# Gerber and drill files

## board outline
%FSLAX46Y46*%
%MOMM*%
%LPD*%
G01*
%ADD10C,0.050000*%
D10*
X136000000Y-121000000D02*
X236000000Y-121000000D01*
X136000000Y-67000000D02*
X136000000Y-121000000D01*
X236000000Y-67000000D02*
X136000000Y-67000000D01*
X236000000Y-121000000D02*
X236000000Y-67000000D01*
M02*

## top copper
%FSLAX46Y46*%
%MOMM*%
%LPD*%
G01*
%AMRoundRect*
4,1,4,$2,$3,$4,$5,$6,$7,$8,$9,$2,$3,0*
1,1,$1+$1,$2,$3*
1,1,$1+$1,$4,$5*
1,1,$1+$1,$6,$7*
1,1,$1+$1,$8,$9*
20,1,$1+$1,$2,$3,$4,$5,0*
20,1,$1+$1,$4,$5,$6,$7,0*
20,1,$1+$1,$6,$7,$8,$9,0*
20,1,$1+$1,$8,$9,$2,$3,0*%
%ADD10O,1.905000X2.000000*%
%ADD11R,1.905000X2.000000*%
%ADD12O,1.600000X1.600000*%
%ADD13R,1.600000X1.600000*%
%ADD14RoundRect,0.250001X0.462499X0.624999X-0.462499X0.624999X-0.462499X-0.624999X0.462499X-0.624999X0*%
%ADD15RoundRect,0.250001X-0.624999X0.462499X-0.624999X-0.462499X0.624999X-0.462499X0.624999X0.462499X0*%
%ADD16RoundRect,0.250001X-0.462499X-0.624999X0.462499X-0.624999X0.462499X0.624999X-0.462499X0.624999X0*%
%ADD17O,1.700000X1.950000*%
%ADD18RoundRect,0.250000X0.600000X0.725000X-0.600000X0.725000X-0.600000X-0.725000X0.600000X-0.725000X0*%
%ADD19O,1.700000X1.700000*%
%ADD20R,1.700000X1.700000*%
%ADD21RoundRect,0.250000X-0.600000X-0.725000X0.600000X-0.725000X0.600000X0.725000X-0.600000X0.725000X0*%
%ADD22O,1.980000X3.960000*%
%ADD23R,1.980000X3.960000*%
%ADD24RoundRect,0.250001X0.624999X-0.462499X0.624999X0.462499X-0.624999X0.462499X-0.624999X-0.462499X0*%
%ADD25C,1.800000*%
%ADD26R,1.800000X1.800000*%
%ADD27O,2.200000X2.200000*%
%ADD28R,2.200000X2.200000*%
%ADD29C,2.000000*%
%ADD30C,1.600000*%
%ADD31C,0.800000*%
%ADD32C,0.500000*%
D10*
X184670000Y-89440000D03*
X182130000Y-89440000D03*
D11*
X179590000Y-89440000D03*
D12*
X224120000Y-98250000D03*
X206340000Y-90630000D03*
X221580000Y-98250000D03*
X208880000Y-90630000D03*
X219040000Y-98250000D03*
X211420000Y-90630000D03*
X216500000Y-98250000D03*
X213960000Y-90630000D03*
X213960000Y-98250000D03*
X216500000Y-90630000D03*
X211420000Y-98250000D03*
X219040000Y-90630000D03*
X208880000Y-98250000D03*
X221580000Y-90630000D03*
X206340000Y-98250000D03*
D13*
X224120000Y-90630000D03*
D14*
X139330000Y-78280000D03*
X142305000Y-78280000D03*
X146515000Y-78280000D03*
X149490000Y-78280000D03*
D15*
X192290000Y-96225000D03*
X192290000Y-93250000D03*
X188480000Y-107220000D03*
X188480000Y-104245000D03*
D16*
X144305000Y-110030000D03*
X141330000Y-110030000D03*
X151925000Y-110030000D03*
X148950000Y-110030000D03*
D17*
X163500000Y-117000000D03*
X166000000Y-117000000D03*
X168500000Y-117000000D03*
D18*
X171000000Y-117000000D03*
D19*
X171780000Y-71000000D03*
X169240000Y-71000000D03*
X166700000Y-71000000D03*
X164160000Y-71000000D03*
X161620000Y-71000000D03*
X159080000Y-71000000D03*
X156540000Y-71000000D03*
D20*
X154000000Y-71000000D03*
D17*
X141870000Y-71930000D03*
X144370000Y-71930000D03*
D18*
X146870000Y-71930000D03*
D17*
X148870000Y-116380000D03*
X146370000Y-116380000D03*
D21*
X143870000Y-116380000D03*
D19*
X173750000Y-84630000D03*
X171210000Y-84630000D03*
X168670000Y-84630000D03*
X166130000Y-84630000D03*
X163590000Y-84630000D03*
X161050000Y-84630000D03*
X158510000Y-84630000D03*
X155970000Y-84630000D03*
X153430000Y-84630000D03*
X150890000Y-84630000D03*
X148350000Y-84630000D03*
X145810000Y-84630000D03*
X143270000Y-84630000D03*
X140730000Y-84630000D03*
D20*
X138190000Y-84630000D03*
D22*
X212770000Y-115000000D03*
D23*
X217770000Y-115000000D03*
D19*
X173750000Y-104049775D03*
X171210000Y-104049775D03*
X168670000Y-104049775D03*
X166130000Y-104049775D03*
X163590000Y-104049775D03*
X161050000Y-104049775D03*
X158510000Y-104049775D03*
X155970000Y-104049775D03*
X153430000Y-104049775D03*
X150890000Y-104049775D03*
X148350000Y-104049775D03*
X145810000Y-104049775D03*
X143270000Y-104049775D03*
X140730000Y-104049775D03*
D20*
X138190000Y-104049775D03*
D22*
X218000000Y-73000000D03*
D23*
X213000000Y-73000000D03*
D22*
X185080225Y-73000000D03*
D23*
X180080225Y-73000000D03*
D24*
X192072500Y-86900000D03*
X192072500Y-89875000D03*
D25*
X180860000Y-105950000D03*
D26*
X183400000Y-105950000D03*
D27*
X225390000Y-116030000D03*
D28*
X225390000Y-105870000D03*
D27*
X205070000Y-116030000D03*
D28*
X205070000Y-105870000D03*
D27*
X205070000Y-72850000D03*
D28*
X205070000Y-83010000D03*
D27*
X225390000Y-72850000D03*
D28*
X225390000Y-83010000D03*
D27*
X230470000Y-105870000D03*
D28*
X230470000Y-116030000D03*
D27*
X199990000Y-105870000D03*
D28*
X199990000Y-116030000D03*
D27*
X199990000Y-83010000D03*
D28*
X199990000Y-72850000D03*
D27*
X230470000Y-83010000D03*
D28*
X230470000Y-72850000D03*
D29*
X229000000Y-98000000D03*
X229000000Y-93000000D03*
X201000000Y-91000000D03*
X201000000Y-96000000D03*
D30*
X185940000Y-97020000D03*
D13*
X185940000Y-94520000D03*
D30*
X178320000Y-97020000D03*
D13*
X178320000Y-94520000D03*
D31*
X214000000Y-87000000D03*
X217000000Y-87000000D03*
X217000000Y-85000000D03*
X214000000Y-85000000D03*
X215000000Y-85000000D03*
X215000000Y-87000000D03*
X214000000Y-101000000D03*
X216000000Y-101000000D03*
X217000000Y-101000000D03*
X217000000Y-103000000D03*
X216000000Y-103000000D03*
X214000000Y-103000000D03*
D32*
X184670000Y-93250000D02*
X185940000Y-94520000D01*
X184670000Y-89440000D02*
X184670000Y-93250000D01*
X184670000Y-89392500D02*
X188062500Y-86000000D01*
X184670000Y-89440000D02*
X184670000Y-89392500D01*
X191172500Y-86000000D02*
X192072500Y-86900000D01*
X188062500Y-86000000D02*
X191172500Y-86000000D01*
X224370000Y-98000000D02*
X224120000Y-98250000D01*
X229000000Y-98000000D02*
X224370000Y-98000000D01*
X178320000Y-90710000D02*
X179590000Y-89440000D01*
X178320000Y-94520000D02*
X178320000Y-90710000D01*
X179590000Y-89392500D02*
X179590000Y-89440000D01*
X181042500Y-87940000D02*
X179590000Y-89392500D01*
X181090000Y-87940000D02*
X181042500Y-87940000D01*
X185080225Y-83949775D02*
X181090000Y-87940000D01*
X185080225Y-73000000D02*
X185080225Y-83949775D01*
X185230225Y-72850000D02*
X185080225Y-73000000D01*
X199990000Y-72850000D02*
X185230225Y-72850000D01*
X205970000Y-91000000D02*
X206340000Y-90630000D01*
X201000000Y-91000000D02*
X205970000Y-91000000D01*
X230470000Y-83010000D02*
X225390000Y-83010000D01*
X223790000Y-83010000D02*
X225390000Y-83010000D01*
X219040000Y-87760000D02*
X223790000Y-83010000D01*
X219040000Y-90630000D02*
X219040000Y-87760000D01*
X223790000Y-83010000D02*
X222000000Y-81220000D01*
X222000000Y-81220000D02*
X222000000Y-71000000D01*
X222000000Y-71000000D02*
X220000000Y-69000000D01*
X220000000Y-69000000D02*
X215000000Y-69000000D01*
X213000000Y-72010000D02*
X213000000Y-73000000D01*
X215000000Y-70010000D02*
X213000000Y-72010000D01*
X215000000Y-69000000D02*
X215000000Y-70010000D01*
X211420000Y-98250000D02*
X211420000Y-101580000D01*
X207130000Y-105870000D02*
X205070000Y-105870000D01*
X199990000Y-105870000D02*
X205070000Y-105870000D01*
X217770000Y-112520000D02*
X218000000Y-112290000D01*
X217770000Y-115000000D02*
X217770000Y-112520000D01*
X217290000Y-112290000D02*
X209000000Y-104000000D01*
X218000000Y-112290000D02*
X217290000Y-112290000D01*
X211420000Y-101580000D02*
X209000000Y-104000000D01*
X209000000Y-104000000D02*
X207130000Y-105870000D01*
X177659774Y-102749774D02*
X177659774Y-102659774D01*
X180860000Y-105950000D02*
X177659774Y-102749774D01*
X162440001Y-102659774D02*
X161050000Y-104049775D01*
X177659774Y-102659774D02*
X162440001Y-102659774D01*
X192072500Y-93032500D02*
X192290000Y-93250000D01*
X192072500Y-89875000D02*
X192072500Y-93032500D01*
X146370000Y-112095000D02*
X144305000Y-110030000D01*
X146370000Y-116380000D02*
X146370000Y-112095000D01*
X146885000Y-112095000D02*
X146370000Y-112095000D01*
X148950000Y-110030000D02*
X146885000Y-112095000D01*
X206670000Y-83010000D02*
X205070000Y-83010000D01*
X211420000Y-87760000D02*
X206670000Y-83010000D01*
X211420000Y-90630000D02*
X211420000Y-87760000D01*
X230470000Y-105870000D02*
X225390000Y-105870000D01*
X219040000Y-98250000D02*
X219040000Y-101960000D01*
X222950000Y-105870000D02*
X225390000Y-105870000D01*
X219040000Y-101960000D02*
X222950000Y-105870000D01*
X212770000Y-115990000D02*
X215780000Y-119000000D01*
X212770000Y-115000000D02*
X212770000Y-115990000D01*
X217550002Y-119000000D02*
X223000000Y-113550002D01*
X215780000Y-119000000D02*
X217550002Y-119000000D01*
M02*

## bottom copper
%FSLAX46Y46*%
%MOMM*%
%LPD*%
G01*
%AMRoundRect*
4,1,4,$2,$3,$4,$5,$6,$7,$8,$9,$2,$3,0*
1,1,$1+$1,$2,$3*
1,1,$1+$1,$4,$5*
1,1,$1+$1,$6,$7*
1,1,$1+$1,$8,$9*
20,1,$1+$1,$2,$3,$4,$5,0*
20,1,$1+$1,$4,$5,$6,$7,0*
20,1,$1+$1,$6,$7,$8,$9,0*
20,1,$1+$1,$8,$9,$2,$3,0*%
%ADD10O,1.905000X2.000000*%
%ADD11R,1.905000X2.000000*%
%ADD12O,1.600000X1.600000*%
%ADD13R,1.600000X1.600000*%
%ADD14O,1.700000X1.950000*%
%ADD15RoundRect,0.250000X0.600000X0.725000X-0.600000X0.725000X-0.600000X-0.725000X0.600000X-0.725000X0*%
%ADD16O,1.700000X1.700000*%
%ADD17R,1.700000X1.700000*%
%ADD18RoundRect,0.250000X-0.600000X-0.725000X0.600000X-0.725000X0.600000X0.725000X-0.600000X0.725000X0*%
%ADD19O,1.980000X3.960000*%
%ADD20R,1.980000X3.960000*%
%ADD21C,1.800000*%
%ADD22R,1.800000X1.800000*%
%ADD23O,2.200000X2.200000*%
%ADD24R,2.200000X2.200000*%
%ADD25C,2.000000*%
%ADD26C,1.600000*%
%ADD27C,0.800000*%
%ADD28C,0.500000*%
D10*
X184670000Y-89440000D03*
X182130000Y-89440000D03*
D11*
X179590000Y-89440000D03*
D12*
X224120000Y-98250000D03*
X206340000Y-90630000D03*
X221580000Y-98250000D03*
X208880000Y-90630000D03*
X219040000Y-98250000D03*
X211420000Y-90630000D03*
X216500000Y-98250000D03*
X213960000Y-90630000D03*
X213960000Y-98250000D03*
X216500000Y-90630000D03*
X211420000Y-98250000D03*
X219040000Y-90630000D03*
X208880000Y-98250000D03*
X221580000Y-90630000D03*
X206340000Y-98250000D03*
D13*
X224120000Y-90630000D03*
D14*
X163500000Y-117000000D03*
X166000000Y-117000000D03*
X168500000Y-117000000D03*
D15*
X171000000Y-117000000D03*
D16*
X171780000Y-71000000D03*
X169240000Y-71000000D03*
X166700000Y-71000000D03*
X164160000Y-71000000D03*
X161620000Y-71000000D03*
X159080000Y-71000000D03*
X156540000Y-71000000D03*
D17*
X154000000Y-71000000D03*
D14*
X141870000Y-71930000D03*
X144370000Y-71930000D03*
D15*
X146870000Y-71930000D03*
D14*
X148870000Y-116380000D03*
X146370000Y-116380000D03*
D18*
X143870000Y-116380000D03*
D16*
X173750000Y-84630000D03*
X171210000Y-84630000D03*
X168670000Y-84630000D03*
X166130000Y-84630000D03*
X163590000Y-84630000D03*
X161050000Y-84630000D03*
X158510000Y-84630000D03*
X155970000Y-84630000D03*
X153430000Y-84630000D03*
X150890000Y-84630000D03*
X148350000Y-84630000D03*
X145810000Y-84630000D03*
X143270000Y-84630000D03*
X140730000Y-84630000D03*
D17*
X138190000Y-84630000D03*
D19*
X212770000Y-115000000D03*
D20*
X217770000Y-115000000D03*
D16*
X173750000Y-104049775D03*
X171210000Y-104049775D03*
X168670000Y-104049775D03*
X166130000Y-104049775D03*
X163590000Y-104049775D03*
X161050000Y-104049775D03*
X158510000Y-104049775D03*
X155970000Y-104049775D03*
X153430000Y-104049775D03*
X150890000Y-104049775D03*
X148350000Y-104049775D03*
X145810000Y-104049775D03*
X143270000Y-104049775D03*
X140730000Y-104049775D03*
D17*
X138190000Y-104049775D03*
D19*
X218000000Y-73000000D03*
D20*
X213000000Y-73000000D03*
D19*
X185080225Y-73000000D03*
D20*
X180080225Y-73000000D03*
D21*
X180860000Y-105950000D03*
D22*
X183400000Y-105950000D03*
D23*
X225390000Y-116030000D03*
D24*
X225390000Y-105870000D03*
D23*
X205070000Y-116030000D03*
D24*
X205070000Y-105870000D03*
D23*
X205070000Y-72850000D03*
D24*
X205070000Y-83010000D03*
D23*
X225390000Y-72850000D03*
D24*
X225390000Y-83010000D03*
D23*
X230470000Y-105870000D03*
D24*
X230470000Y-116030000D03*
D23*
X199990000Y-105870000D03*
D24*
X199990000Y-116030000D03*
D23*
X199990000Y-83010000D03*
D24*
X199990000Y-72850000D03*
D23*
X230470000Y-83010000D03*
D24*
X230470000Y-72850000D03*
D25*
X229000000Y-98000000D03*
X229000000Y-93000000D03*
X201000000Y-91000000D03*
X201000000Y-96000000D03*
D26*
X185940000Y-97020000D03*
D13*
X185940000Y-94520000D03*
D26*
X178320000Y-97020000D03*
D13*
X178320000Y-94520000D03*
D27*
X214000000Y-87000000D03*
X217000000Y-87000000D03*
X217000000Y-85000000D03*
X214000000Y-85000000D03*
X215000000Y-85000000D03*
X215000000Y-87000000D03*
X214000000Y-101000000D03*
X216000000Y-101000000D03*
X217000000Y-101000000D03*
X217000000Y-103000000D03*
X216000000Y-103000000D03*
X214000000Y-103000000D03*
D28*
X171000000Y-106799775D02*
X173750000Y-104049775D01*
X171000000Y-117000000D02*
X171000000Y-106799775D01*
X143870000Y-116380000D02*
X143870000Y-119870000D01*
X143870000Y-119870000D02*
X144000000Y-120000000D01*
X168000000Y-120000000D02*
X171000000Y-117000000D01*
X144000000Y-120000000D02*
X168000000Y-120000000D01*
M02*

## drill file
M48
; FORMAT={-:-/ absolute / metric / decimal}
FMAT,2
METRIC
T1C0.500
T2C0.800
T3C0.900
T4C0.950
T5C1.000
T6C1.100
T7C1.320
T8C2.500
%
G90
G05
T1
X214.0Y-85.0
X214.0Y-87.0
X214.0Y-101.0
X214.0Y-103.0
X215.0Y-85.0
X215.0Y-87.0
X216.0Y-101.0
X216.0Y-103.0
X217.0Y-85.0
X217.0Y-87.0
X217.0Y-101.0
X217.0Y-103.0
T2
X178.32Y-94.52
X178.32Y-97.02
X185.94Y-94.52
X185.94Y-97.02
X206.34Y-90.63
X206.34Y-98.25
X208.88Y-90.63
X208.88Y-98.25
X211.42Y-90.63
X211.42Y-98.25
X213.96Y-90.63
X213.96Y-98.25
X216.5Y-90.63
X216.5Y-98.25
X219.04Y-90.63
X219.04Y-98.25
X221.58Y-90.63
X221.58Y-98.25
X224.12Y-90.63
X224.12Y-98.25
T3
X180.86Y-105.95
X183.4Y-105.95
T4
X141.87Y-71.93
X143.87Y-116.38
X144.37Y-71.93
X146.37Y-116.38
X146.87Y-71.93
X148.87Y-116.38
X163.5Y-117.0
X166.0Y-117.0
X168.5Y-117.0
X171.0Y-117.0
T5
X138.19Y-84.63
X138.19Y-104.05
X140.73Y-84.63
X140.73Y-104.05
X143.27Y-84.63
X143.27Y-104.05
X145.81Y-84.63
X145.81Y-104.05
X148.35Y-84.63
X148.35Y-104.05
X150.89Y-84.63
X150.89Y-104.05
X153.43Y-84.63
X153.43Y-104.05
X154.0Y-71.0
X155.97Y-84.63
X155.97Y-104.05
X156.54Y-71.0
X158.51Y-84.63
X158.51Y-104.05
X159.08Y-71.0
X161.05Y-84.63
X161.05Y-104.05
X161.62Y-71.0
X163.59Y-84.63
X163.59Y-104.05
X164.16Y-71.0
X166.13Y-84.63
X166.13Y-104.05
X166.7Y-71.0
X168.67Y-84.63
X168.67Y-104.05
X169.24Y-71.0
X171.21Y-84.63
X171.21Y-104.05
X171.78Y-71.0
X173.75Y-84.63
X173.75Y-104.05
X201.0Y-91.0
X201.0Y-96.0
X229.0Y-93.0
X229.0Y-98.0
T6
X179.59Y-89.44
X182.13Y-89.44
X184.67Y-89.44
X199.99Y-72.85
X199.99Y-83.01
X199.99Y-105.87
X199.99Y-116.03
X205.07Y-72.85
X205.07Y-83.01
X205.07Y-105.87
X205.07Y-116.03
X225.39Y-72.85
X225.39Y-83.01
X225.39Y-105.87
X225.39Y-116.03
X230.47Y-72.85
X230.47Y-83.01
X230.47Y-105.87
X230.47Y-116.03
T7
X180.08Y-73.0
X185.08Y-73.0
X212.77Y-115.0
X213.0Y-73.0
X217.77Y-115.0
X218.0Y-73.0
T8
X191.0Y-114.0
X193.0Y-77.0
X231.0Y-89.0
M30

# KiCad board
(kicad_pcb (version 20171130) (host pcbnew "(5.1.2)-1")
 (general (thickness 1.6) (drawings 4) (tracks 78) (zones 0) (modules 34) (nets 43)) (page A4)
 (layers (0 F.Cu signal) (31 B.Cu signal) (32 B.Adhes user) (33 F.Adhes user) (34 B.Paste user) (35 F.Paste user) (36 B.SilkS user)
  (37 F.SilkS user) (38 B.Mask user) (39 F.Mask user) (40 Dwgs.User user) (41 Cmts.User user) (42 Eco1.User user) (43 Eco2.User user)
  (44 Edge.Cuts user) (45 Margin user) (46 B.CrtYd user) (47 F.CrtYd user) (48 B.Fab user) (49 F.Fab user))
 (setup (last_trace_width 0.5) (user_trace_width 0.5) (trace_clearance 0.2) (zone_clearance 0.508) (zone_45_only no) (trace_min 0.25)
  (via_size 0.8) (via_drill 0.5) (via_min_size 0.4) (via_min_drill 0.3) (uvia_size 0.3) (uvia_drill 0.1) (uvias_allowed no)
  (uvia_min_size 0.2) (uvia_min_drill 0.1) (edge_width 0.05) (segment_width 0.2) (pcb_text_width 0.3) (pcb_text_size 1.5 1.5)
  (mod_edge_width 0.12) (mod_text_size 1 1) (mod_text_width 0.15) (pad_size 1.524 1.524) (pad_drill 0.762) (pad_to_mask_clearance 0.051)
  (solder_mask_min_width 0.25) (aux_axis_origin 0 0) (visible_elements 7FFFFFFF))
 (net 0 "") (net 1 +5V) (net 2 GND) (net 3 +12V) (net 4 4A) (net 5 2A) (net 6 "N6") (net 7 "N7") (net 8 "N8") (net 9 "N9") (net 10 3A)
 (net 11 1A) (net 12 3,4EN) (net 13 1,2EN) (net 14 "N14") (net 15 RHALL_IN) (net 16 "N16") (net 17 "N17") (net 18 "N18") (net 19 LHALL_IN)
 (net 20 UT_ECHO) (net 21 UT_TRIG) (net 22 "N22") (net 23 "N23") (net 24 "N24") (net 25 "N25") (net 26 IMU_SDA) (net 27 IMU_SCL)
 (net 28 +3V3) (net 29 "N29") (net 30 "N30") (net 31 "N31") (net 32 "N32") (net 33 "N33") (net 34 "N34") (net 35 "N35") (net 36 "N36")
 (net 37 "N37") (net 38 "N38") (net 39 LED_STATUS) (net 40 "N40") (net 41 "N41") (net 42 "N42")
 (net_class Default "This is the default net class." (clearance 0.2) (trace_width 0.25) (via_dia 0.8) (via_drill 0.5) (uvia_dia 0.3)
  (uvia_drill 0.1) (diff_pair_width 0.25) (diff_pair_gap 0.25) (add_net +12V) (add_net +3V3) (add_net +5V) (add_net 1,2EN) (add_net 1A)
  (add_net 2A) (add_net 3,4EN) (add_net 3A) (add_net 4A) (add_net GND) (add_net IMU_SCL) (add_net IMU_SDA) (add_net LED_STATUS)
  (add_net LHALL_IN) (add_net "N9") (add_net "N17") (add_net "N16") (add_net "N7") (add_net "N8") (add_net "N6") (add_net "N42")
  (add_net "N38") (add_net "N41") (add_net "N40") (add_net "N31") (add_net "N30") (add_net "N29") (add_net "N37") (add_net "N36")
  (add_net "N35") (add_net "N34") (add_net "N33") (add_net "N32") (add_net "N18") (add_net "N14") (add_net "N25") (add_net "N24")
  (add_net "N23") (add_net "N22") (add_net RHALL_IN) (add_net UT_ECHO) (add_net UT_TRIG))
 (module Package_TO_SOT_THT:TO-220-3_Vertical (layer F.Cu) (at 179.59 89.44)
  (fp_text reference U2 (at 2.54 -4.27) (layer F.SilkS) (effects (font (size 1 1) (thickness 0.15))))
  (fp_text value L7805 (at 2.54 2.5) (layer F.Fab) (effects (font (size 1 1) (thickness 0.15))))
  (pad 3 thru_hole oval (at 5.08 0) (size 1.905 2) (drill 1.1) (layers *.Cu *.Mask) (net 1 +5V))
  (pad 2 thru_hole oval (at 2.54 0) (size 1.905 2) (drill 1.1) (layers *.Cu *.Mask) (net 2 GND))
  (pad 1 thru_hole rect (at 0 0) (size 1.905 2) (drill 1.1) (layers *.Cu *.Mask) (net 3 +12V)))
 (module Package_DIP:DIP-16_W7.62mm (layer F.Cu) (at 224.12 90.63 270)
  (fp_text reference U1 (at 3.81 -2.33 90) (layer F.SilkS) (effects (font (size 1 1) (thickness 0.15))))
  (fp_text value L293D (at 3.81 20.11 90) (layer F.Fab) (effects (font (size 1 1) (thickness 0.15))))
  (pad 16 thru_hole oval (at 7.62 0 270) (size 1.6 1.6) (drill 0.8) (layers *.Cu *.Mask) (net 1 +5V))
  (pad 8 thru_hole oval (at 0 17.78 270) (size 1.6 1.6) (drill 0.8) (layers *.Cu *.Mask) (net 3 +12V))
  (pad 15 thru_hole oval (at 7.62 2.54 270) (size 1.6 1.6) (drill 0.8) (layers *.Cu *.Mask) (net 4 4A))
  (pad 7 thru_hole oval (at 0 15.24 270) (size 1.6 1.6) (drill 0.8) (layers *.Cu *.Mask) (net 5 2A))
  (pad 14 thru_hole oval (at 7.62 5.08 270) (size 1.6 1.6) (drill 0.8) (layers *.Cu *.Mask) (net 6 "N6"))
  (pad 6 thru_hole oval (at 0 12.7 270) (size 1.6 1.6) (drill 0.8) (layers *.Cu *.Mask) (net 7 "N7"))
  (pad 13 thru_hole oval (at 7.62 7.62 270) (size 1.6 1.6) (drill 0.8) (layers *.Cu *.Mask) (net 2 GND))
  (pad 5 thru_hole oval (at 0 10.16 270) (size 1.6 1.6) (drill 0.8) (layers *.Cu *.Mask) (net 2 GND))
  (pad 12 thru_hole oval (at 7.62 10.16 270) (size 1.6 1.6) (drill 0.8) (layers *.Cu *.Mask) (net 2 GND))
  (pad 4 thru_hole oval (at 0 7.62 270) (size 1.6 1.6) (drill 0.8) (layers *.Cu *.Mask) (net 2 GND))
  (pad 11 thru_hole oval (at 7.62 12.7 270) (size 1.6 1.6) (drill 0.8) (layers *.Cu *.Mask) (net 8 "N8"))
  (pad 3 thru_hole oval (at 0 5.08 270) (size 1.6 1.6) (drill 0.8) (layers *.Cu *.Mask) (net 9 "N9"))
  (pad 10 thru_hole oval (at 7.62 15.24 270) (size 1.6 1.6) (drill 0.8) (layers *.Cu *.Mask) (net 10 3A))
  (pad 2 thru_hole oval (at 0 2.54 270) (size 1.6 1.6) (drill 0.8) (layers *.Cu *.Mask) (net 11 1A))
  (pad 9 thru_hole oval (at 7.62 17.78 270) (size 1.6 1.6) (drill 0.8) (layers *.Cu *.Mask) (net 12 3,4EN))
  (pad 1 thru_hole rect (at 0 0 270) (size 1.6 1.6) (drill 0.8) (layers *.Cu *.Mask) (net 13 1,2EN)))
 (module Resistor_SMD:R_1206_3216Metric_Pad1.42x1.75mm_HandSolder (layer F.Cu) (at 140.8175 78.28 180)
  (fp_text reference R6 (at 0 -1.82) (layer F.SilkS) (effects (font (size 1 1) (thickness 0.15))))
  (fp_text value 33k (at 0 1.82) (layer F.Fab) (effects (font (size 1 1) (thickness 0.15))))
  (pad 2 smd roundrect (at 1.4875 0 180) (size 1.425 1.75) (layers F.Cu F.Paste F.Mask) (roundrect_rratio 0.175439) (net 2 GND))
  (pad 1 smd roundrect (at -1.4875 0 180) (size 1.425 1.75) (layers F.Cu F.Paste F.Mask) (roundrect_rratio 0.175439) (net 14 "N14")))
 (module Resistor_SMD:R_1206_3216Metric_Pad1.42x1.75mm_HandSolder (layer F.Cu) (at 148.0025 78.28 180)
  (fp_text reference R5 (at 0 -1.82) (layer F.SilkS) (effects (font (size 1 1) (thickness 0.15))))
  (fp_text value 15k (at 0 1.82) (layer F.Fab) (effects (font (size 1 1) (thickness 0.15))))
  (pad 2 smd roundrect (at 1.4875 0 180) (size 1.425 1.75) (layers F.Cu F.Paste F.Mask) (roundrect_rratio 0.175439) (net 14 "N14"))
  (pad 1 smd roundrect (at -1.4875 0 180) (size 1.425 1.75) (layers F.Cu F.Paste F.Mask) (roundrect_rratio 0.175439) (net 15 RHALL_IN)))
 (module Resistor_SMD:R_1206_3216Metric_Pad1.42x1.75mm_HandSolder (layer F.Cu) (at 192.29 94.7375 270)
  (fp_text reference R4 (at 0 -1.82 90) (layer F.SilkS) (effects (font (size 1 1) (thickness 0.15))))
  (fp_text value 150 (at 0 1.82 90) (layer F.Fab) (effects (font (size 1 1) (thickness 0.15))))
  (pad 2 smd roundrect (at 1.4875 0 270) (size 1.425 1.75) (layers F.Cu F.Paste F.Mask) (roundrect_rratio 0.175439) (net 2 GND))
  (pad 1 smd roundrect (at -1.4875 0 270) (size 1.425 1.75) (layers F.Cu F.Paste F.Mask) (roundrect_rratio 0.175439) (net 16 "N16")))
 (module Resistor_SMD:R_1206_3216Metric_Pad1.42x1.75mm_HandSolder (layer F.Cu) (at 188.48 105.7325 270)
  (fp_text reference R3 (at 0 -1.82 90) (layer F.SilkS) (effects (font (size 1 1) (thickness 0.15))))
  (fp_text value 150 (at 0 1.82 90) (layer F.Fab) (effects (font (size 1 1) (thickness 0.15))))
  (pad 2 smd roundrect (at 1.4875 0 270) (size 1.425 1.75) (layers F.Cu F.Paste F.Mask) (roundrect_rratio 0.175439) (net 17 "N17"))
  (pad 1 smd roundrect (at -1.4875 0 270) (size 1.425 1.75) (layers F.Cu F.Paste F.Mask) (roundrect_rratio 0.175439) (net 2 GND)))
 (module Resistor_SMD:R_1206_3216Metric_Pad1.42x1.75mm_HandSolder (layer F.Cu) (at 142.8175 110.03)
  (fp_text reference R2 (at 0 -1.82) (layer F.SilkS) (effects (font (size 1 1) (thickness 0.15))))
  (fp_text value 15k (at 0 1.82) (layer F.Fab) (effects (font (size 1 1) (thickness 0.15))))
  (pad 2 smd roundrect (at 1.4875 0) (size 1.425 1.75) (layers F.Cu F.Paste F.Mask) (roundrect_rratio 0.175439) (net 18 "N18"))
  (pad 1 smd roundrect (at -1.4875 0) (size 1.425 1.75) (layers F.Cu F.Paste F.Mask) (roundrect_rratio 0.175439) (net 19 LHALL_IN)))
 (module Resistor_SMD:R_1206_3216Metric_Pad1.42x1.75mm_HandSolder (layer F.Cu) (at 150.4375 110.03)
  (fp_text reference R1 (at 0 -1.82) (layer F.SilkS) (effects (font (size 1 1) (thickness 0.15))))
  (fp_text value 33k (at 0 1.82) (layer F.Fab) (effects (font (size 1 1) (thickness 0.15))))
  (pad 2 smd roundrect (at 1.4875 0) (size 1.425 1.75) (layers F.Cu F.Paste F.Mask) (roundrect_rratio 0.175439) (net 2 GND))
  (pad 1 smd roundrect (at -1.4875 0) (size 1.425 1.75) (layers F.Cu F.Paste F.Mask) (roundrect_rratio 0.175439) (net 18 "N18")))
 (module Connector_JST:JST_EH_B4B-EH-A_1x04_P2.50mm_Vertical (layer F.Cu) (at 171 117 180)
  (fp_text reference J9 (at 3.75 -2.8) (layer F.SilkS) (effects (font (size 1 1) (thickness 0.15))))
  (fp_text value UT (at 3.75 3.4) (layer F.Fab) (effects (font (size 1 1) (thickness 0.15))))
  (pad 4 thru_hole oval (at 7.5 0 180) (size 1.7 1.95) (drill 0.95) (layers *.Cu *.Mask) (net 2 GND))
  (pad 3 thru_hole oval (at 5 0 180) (size 1.7 1.95) (drill 0.95) (layers *.Cu *.Mask) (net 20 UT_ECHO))
  (pad 2 thru_hole oval (at 2.5 0 180) (size 1.7 1.95) (drill 0.95) (layers *.Cu *.Mask) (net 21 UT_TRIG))
  (pad 1 thru_hole roundrect (at 0 0 180) (size 1.7 1.95) (drill 0.95) (layers *.Cu *.Mask) (roundrect_rratio 0.147059) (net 1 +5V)))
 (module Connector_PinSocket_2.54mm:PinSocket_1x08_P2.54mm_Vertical (layer F.Cu) (at 154 71 90)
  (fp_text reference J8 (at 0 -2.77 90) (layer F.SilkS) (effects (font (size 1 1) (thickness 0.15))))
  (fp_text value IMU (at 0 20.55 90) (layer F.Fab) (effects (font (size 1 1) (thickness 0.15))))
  (pad 8 thru_hole oval (at 0 17.78 90) (size 1.7 1.7) (drill 1) (layers *.Cu *.Mask) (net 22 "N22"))
  (pad 7 thru_hole oval (at 0 15.24 90) (size 1.7 1.7) (drill 1) (layers *.Cu *.Mask) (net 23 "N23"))
  (pad 6 thru_hole oval (at 0 12.7 90) (size 1.7 1.7) (drill 1) (layers *.Cu *.Mask) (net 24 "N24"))
  (pad 5 thru_hole oval (at 0 10.16 90) (size 1.7 1.7) (drill 1) (layers *.Cu *.Mask) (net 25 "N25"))
  (pad 4 thru_hole oval (at 0 7.62 90) (size 1.7 1.7) (drill 1) (layers *.Cu *.Mask) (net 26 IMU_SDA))
  (pad 3 thru_hole oval (at 0 5.08 90) (size 1.7 1.7) (drill 1) (layers *.Cu *.Mask) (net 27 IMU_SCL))
  (pad 2 thru_hole oval (at 0 2.54 90) (size 1.7 1.7) (drill 1) (layers *.Cu *.Mask) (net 2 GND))
  (pad 1 thru_hole rect (at 0 0 90) (size 1.7 1.7) (drill 1) (layers *.Cu *.Mask) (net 1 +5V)))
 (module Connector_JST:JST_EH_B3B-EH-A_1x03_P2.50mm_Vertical (layer F.Cu) (at 146.87 71.93 180)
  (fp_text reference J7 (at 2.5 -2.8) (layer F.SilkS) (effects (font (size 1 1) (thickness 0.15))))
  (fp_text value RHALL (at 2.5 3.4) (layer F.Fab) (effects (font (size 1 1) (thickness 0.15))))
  (pad 3 thru_hole oval (at 5 0 180) (size 1.7 1.95) (drill 0.95) (layers *.Cu *.Mask) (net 2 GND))
  (pad 2 thru_hole oval (at 2.5 0 180) (size 1.7 1.95) (drill 0.95) (layers *.Cu *.Mask) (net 14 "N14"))
  (pad 1 thru_hole roundrect (at 0 0 180) (size 1.7 1.95) (drill 0.95) (layers *.Cu *.Mask) (roundrect_rratio 0.147059) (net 1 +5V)))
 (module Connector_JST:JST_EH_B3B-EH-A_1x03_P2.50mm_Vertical (layer F.Cu) (at 143.87 116.38)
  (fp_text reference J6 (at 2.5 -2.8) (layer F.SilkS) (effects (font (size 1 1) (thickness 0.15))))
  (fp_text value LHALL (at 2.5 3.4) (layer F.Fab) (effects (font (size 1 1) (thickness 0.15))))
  (pad 3 thru_hole oval (at 5 0) (size 1.7 1.95) (drill 0.95) (layers *.Cu *.Mask) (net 2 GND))
  (pad 2 thru_hole oval (at 2.5 0) (size 1.7 1.95) (drill 0.95) (layers *.Cu *.Mask) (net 18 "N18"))
  (pad 1 thru_hole roundrect (at 0 0) (size 1.7 1.95) (drill 0.95) (layers *.Cu *.Mask) (roundrect_rratio 0.147059) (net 1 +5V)))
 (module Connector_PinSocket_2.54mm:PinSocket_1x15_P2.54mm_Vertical (layer F.Cu) (at 138.19 84.63 90)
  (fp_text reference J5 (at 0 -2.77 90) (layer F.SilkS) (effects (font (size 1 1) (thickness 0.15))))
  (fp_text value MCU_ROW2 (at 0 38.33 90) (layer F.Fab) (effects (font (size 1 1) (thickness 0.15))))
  (pad 15 thru_hole oval (at 0 35.56 90) (size 1.7 1.7) (drill 1) (layers *.Cu *.Mask) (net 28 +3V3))
  (pad 14 thru_hole oval (at 0 33.02 90) (size 1.7 1.7) (drill 1) (layers *.Cu *.Mask) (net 2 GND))
  (pad 13 thru_hole oval (at 0 30.48 90) (size 1.7 1.7) (drill 1) (layers *.Cu *.Mask) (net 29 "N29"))
  (pad 12 thru_hole oval (at 0 27.94 90) (size 1.7 1.7) (drill 1) (layers *.Cu *.Mask) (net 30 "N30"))
  (pad 11 thru_hole oval (at 0 25.4 90) (size 1.7 1.7) (drill 1) (layers *.Cu *.Mask) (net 21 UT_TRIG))
  (pad 10 thru_hole oval (at 0 22.86 90) (size 1.7 1.7) (drill 1) (layers *.Cu *.Mask) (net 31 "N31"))
  (pad 9 thru_hole oval (at 0 20.32 90) (size 1.7 1.7) (drill 1) (layers *.Cu *.Mask) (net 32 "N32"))
  (pad 8 thru_hole oval (at 0 17.78 90) (size 1.7 1.7) (drill 1) (layers *.Cu *.Mask) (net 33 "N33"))
  (pad 7 thru_hole oval (at 0 15.24 90) (size 1.7 1.7) (drill 1) (layers *.Cu *.Mask) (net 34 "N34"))
  (pad 6 thru_hole oval (at 0 12.7 90) (size 1.7 1.7) (drill 1) (layers *.Cu *.Mask) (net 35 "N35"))
  (pad 5 thru_hole oval (at 0 10.16 90) (size 1.7 1.7) (drill 1) (layers *.Cu *.Mask) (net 26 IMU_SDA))
  (pad 4 thru_hole oval (at 0 7.62 90) (size 1.7 1.7) (drill 1) (layers *.Cu *.Mask) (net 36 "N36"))
  (pad 3 thru_hole oval (at 0 5.08 90) (size 1.7 1.7) (drill 1) (layers *.Cu *.Mask) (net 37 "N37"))
  (pad 2 thru_hole oval (at 0 2.54 90) (size 1.7 1.7) (drill 1) (layers *.Cu *.Mask) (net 27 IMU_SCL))
  (pad 1 thru_hole rect (at 0 0 90) (size 1.7 1.7) (drill 1) (layers *.Cu *.Mask) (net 20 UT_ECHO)))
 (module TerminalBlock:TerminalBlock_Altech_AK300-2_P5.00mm (layer F.Cu) (at 217.77 115 180)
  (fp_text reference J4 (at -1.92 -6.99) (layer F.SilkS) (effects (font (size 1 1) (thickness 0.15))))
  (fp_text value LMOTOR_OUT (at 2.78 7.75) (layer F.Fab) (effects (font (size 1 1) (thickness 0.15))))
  (pad 2 thru_hole oval (at 5 0 180) (size 1.98 3.96) (drill 1.32) (layers *.Cu *.Mask) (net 6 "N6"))
  (pad 1 thru_hole rect (at 0 0 180) (size 1.98 3.96) (drill 1.32) (layers *.Cu *.Mask) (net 8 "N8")))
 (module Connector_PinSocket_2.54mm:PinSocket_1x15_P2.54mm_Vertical (layer F.Cu) (at 138.19 104.049775 90)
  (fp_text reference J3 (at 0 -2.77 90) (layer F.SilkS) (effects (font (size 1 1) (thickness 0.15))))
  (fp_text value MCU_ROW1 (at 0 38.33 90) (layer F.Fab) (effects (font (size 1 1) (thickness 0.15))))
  (pad 15 thru_hole oval (at 0 35.56 90) (size 1.7 1.7) (drill 1) (layers *.Cu *.Mask) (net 1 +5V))
  (pad 14 thru_hole oval (at 0 33.02 90) (size 1.7 1.7) (drill 1) (layers *.Cu *.Mask) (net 2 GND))
  (pad 13 thru_hole oval (at 0 30.48 90) (size 1.7 1.7) (drill 1) (layers *.Cu *.Mask) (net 4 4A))
  (pad 12 thru_hole oval (at 0 27.94 90) (size 1.7 1.7) (drill 1) (layers *.Cu *.Mask) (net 5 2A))
  (pad 11 thru_hole oval (at 0 25.4 90) (size 1.7 1.7) (drill 1) (layers *.Cu *.Mask) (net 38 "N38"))
  (pad 10 thru_hole oval (at 0 22.86 90) (size 1.7 1.7) (drill 1) (layers *.Cu *.Mask) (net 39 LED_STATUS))
  (pad 9 thru_hole oval (at 0 20.32 90) (size 1.7 1.7) (drill 1) (layers *.Cu *.Mask) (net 12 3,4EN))
  (pad 8 thru_hole oval (at 0 17.78 90) (size 1.7 1.7) (drill 1) (layers *.Cu *.Mask) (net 10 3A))
  (pad 7 thru_hole oval (at 0 15.24 90) (size 1.7 1.7) (drill 1) (layers *.Cu *.Mask) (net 13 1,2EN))
  (pad 6 thru_hole oval (at 0 12.7 90) (size 1.7 1.7) (drill 1) (layers *.Cu *.Mask) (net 11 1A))
  (pad 5 thru_hole oval (at 0 10.16 90) (size 1.7 1.7) (drill 1) (layers *.Cu *.Mask) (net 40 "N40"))
  (pad 4 thru_hole oval (at 0 7.62 90) (size 1.7 1.7) (drill 1) (layers *.Cu *.Mask) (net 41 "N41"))
  (pad 3 thru_hole oval (at 0 5.08 90) (size 1.7 1.7) (drill 1) (layers *.Cu *.Mask) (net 19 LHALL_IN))
  (pad 2 thru_hole oval (at 0 2.54 90) (size 1.7 1.7) (drill 1) (layers *.Cu *.Mask) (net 15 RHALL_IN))
  (pad 1 thru_hole rect (at 0 0 90) (size 1.7 1.7) (drill 1) (layers *.Cu *.Mask) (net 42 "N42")))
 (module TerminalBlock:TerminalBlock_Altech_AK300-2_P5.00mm (layer F.Cu) (at 213 73)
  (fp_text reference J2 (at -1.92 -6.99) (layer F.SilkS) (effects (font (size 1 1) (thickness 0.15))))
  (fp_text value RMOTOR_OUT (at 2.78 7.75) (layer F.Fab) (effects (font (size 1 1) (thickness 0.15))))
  (pad 2 thru_hole oval (at 5 0) (size 1.98 3.96) (drill 1.32) (layers *.Cu *.Mask) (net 7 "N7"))
  (pad 1 thru_hole rect (at 0 0) (size 1.98 3.96) (drill 1.32) (layers *.Cu *.Mask) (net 9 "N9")))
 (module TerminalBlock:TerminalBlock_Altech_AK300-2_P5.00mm (layer F.Cu) (at 180.080225 73)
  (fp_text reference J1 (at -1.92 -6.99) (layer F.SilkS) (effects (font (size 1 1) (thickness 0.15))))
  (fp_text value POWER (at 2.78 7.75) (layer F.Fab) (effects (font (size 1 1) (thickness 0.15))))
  (pad 2 thru_hole oval (at 5 0) (size 1.98 3.96) (drill 1.32) (layers *.Cu *.Mask) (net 3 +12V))
  (pad 1 thru_hole rect (at 0 0) (size 1.98 3.96) (drill 1.32) (layers *.Cu *.Mask) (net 2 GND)))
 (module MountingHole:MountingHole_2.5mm (layer F.Cu) (at 231 89)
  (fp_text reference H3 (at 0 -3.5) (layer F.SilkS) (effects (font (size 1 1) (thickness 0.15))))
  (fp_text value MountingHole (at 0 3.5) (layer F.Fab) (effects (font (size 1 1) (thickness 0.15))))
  (pad 1 np_thru_hole circle (at 0 0) (size 2.5 2.5) (drill 2.5) (layers *.Cu *.Mask)))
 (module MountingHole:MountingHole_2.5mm (layer F.Cu) (at 193 77)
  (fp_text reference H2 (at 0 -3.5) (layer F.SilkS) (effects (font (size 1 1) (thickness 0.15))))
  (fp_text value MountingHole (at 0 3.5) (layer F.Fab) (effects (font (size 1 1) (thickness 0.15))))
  (pad 1 np_thru_hole circle (at 0 0) (size 2.5 2.5) (drill 2.5) (layers *.Cu *.Mask)))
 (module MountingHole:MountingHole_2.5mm (layer F.Cu) (at 191 114)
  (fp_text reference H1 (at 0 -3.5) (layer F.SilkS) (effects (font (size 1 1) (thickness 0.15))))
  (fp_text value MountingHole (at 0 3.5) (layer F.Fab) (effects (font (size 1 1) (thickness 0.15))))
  (pad 1 np_thru_hole circle (at 0 0) (size 2.5 2.5) (drill 2.5) (layers *.Cu *.Mask)))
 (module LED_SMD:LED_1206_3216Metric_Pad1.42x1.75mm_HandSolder (layer F.Cu) (at 192.0725 88.3875 90)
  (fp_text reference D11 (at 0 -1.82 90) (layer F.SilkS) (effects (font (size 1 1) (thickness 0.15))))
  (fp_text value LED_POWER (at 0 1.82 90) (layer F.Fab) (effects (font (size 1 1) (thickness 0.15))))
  (pad 2 smd roundrect (at 1.4875 0 90) (size 1.425 1.75) (layers F.Cu F.Paste F.Mask) (roundrect_rratio 0.175439) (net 1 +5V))
  (pad 1 smd roundrect (at -1.4875 0 90) (size 1.425 1.75) (layers F.Cu F.Paste F.Mask) (roundrect_rratio 0.175439) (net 16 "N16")))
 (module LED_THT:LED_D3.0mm (layer F.Cu) (at 183.4 105.95 180)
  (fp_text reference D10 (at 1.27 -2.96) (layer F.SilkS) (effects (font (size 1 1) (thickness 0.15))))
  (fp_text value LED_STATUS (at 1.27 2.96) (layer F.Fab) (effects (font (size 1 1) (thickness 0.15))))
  (pad 2 thru_hole circle (at 2.54 0 180) (size 1.8 1.8) (drill 0.9) (layers *.Cu *.Mask) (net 39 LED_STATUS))
  (pad 1 thru_hole rect (at 0 0 180) (size 1.8 1.8) (drill 0.9) (layers *.Cu *.Mask) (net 17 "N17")))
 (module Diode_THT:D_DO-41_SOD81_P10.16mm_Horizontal (layer F.Cu) (at 225.39 105.87 270)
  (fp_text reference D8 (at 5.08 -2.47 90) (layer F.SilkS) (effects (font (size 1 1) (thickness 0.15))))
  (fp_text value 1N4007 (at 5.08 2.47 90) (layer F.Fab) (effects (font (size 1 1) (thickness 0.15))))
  (pad 2 thru_hole oval (at 10.16 0 270) (size 2.2 2.2) (drill 1.1) (layers *.Cu *.Mask) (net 2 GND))
  (pad 1 thru_hole rect (at 0 0 270) (size 2.2 2.2) (drill 1.1) (layers *.Cu *.Mask) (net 6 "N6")))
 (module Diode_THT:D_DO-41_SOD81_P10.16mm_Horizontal (layer F.Cu) (at 205.07 105.87 270)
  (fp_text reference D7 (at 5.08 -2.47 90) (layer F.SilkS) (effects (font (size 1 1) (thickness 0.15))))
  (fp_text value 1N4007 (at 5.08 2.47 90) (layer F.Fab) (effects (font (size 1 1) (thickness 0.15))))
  (pad 2 thru_hole oval (at 10.16 0 270) (size 2.2 2.2) (drill 1.1) (layers *.Cu *.Mask) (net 2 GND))
  (pad 1 thru_hole rect (at 0 0 270) (size 2.2 2.2) (drill 1.1) (layers *.Cu *.Mask) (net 8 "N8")))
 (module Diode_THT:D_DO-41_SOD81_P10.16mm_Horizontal (layer F.Cu) (at 205.07 83.01 90)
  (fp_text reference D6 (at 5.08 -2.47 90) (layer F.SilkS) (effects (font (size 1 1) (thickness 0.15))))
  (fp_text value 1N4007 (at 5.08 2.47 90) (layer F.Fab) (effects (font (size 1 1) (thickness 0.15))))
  (pad 2 thru_hole oval (at 10.16 0 90) (size 2.2 2.2) (drill 1.1) (layers *.Cu *.Mask) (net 2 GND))
  (pad 1 thru_hole rect (at 0 0 90) (size 2.2 2.2) (drill 1.1) (layers *.Cu *.Mask) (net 7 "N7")))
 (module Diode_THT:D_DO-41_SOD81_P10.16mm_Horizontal (layer F.Cu) (at 225.39 83.01 90)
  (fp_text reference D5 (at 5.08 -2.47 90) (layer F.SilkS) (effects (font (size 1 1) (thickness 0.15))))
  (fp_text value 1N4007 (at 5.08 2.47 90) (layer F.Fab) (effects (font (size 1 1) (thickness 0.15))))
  (pad 2 thru_hole oval (at 10.16 0 90) (size 2.2 2.2) (drill 1.1) (layers *.Cu *.Mask) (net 2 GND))
  (pad 1 thru_hole rect (at 0 0 90) (size 2.2 2.2) (drill 1.1) (layers *.Cu *.Mask) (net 9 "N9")))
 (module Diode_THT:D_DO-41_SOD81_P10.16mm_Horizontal (layer F.Cu) (at 230.47 116.03 90)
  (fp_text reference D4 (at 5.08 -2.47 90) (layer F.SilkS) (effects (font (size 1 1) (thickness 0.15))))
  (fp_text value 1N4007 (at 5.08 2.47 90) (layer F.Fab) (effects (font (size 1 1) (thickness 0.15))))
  (pad 2 thru_hole oval (at 10.16 0 90) (size 2.2 2.2) (drill 1.1) (layers *.Cu *.Mask) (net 6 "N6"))
  (pad 1 thru_hole rect (at 0 0 90) (size 2.2 2.2) (drill 1.1) (layers *.Cu *.Mask) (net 3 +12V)))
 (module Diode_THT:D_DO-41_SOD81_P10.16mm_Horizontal (layer F.Cu) (at 199.99 116.03 90)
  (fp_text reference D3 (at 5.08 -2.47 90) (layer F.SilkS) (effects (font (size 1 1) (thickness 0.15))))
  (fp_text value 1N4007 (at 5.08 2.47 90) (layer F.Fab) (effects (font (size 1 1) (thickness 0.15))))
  (pad 2 thru_hole oval (at 10.16 0 90) (size 2.2 2.2) (drill 1.1) (layers *.Cu *.Mask) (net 8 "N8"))
  (pad 1 thru_hole rect (at 0 0 90) (size 2.2 2.2) (drill 1.1) (layers *.Cu *.Mask) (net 3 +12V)))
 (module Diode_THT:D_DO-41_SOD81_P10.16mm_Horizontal (layer F.Cu) (at 199.99 72.85 270)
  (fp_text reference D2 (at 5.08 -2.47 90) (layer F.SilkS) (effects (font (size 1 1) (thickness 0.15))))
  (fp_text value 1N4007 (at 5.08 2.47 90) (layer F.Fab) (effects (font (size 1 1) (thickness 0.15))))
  (pad 2 thru_hole oval (at 10.16 0 270) (size 2.2 2.2) (drill 1.1) (layers *.Cu *.Mask) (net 7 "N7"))
  (pad 1 thru_hole rect (at 0 0 270) (size 2.2 2.2) (drill 1.1) (layers *.Cu *.Mask) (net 3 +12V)))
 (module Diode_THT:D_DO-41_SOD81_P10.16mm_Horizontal (layer F.Cu) (at 230.47 72.85 270)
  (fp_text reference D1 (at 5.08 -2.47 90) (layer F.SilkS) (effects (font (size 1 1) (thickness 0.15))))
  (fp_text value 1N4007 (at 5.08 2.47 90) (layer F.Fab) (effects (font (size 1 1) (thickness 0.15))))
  (pad 2 thru_hole oval (at 10.16 0 270) (size 2.2 2.2) (drill 1.1) (layers *.Cu *.Mask) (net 9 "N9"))
  (pad 1 thru_hole rect (at 0 0 270) (size 2.2 2.2) (drill 1.1) (layers *.Cu *.Mask) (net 3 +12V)))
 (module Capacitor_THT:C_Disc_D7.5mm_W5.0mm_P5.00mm (layer F.Cu) (at 229 93 270)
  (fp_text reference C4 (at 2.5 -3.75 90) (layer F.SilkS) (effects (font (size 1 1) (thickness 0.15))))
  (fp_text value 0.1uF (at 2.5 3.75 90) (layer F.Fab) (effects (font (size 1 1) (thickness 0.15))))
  (pad 2 thru_hole circle (at 5 0 270) (size 2 2) (drill 1) (layers *.Cu *.Mask) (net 1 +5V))
  (pad 1 thru_hole circle (at 0 0 270) (size 2 2) (drill 1) (layers *.Cu *.Mask) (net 2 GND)))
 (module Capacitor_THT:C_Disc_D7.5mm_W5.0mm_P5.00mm (layer F.Cu) (at 201 96 90)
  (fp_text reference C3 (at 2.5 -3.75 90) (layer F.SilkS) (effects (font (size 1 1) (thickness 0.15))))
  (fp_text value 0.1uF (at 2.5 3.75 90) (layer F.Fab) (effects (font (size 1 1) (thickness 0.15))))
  (pad 2 thru_hole circle (at 5 0 90) (size 2 2) (drill 1) (layers *.Cu *.Mask) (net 3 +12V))
  (pad 1 thru_hole circle (at 0 0 90) (size 2 2) (drill 1) (layers *.Cu *.Mask) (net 2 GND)))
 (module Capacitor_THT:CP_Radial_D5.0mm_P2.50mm (layer F.Cu) (at 185.94 94.52 270)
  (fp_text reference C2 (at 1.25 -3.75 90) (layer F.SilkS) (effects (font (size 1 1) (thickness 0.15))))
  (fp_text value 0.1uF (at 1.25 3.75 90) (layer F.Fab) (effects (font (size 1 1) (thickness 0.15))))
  (pad 2 thru_hole circle (at 2.5 0 270) (size 1.6 1.6) (drill 0.8) (layers *.Cu *.Mask) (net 2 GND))
  (pad 1 thru_hole rect (at 0 0 270) (size 1.6 1.6) (drill 0.8) (layers *.Cu *.Mask) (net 1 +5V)))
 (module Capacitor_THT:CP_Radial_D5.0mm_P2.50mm (layer F.Cu) (at 178.32 94.52 270)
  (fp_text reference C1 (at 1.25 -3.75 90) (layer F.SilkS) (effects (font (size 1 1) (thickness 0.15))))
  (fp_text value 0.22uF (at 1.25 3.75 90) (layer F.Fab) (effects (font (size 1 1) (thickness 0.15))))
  (pad 2 thru_hole circle (at 2.5 0 270) (size 1.6 1.6) (drill 0.8) (layers *.Cu *.Mask) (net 2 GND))
  (pad 1 thru_hole rect (at 0 0 270) (size 1.6 1.6) (drill 0.8) (layers *.Cu *.Mask) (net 3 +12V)))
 (gr_line (start 136 121) (end 236 121) (layer Edge.Cuts) (width 0.05))
 (gr_line (start 136 67) (end 136 121) (layer Edge.Cuts) (width 0.05))
 (gr_line (start 236 67) (end 136 67) (layer Edge.Cuts) (width 0.05))
 (gr_line (start 236 121) (end 236 67) (layer Edge.Cuts) (width 0.05))
 (via (at 214 87) (size 0.8) (drill 0.5) (layers F.Cu B.Cu) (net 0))
 (via (at 217 87) (size 0.8) (drill 0.5) (layers F.Cu B.Cu) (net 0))
 (via (at 217 85) (size 0.8) (drill 0.5) (layers F.Cu B.Cu) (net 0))
 (via (at 214 85) (size 0.8) (drill 0.5) (layers F.Cu B.Cu) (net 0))
 (via (at 215 85) (size 0.8) (drill 0.5) (layers F.Cu B.Cu) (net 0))
 (via (at 215 87) (size 0.8) (drill 0.5) (layers F.Cu B.Cu) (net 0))
 (via (at 214 101) (size 0.8) (drill 0.5) (layers F.Cu B.Cu) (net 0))
 (via (at 216 101) (size 0.8) (drill 0.5) (layers F.Cu B.Cu) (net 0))
 (via (at 217 101) (size 0.8) (drill 0.5) (layers F.Cu B.Cu) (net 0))
 (via (at 217 103) (size 0.8) (drill 0.5) (layers F.Cu B.Cu) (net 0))
 (via (at 216 103) (size 0.8) (drill 0.5) (layers F.Cu B.Cu) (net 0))
 (via (at 214 103) (size 0.8) (drill 0.5) (layers F.Cu B.Cu) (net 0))
 (segment (start 184.67 93.25) (end 185.94 94.52) (width 0.5) (layer F.Cu) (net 1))
 (segment (start 184.67 89.44) (end 184.67 93.25) (width 0.5) (layer F.Cu) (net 1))
 (segment (start 184.67 89.3925) (end 188.0625 86) (width 0.5) (layer F.Cu) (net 1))
 (segment (start 184.67 89.44) (end 184.67 89.3925) (width 0.5) (layer F.Cu) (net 1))
 (segment (start 191.1725 86) (end 192.0725 86.9) (width 0.5) (layer F.Cu) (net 1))
 (segment (start 188.0625 86) (end 191.1725 86) (width 0.5) (layer F.Cu) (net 1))
 (segment (start 171 106.799775) (end 173.75 104.049775) (width 0.5) (layer B.Cu) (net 1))
 (segment (start 171 117) (end 171 106.799775) (width 0.5) (layer B.Cu) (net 1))
 (segment (start 143.87 116.38) (end 143.87 119.87) (width 0.5) (layer B.Cu) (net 1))
 (segment (start 143.87 119.87) (end 144 120) (width 0.5) (layer B.Cu) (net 1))
 (segment (start 168 120) (end 171 117) (width 0.5) (layer B.Cu) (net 1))
 (segment (start 144 120) (end 168 120) (width 0.5) (layer B.Cu) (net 1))
 (segment (start 224.37 98) (end 224.12 98.25) (width 0.5) (layer F.Cu) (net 1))
 (segment (start 229 98) (end 224.37 98) (width 0.5) (layer F.Cu) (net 1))
 (segment (start 178.32 90.71) (end 179.59 89.44) (width 0.5) (layer F.Cu) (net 3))
 (segment (start 178.32 94.52) (end 178.32 90.71) (width 0.5) (layer F.Cu) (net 3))
 (segment (start 179.59 89.3925) (end 179.59 89.44) (width 0.5) (layer F.Cu) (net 3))
 (segment (start 181.0425 87.94) (end 179.59 89.3925) (width 0.5) (layer F.Cu) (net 3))
 (segment (start 181.09 87.94) (end 181.0425 87.94) (width 0.5) (layer F.Cu) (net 3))
 (segment (start 185.080225 83.949775) (end 181.09 87.94) (width 0.5) (layer F.Cu) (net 3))
 (segment (start 185.080225 73) (end 185.080225 83.949775) (width 0.5) (layer F.Cu) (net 3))
 (segment (start 185.230225 72.85) (end 185.080225 73) (width 0.5) (layer F.Cu) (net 3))
 (segment (start 199.99 72.85) (end 185.230225 72.85) (width 0.5) (layer F.Cu) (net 3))
 (segment (start 205.97 91) (end 206.34 90.63) (width 0.5) (layer F.Cu) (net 3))
 (segment (start 201 91) (end 205.97 91) (width 0.5) (layer F.Cu) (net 3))
 (segment (start 230.47 83.01) (end 225.39 83.01) (width 0.5) (layer F.Cu) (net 9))
 (segment (start 223.79 83.01) (end 225.39 83.01) (width 0.5) (layer F.Cu) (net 9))
 (segment (start 219.04 87.76) (end 223.79 83.01) (width 0.5) (layer F.Cu) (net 9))
 (segment (start 219.04 90.63) (end 219.04 87.76) (width 0.5) (layer F.Cu) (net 9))
 (segment (start 223.79 83.01) (end 222 81.22) (width 0.5) (layer F.Cu) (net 9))
 (segment (start 222 81.22) (end 222 71) (width 0.5) (layer F.Cu) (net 9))
 (segment (start 222 71) (end 220 69) (width 0.5) (layer F.Cu) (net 9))
 (segment (start 220 69) (end 215 69) (width 0.5) (layer F.Cu) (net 9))
 (segment (start 213 72.01) (end 213 73) (width 0.5) (layer F.Cu) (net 9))
 (segment (start 215 70.01) (end 213 72.01) (width 0.5) (layer F.Cu) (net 9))
 (segment (start 215 69) (end 215 70.01) (width 0.5) (layer F.Cu) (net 9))
 (segment (start 211.42 98.25) (end 211.42 101.58) (width 0.5) (layer F.Cu) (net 8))
 (segment (start 207.13 105.87) (end 205.07 105.87) (width 0.5) (layer F.Cu) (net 8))
 (segment (start 199.99 105.87) (end 205.07 105.87) (width 0.5) (layer F.Cu) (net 8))
 (segment (start 217.77 112.52) (end 218 112.29) (width 0.5) (layer F.Cu) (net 8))
 (segment (start 217.77 115) (end 217.77 112.52) (width 0.5) (layer F.Cu) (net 8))
 (segment (start 217.29 112.29) (end 209 104) (width 0.5) (layer F.Cu) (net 8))
 (segment (start 218 112.29) (end 217.29 112.29) (width 0.5) (layer F.Cu) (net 8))
 (segment (start 211.42 101.58) (end 209 104) (width 0.5) (layer F.Cu) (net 8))
 (segment (start 209 104) (end 207.13 105.87) (width 0.5) (layer F.Cu) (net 8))
 (segment (start 177.659774 102.749774) (end 177.659774 102.659774) (width 0.5) (layer F.Cu) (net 39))
 (segment (start 180.86 105.95) (end 177.659774 102.749774) (width 0.5) (layer F.Cu) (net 39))
 (segment (start 162.440001 102.659774) (end 161.05 104.049775) (width 0.5) (layer F.Cu) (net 39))
 (segment (start 177.659774 102.659774) (end 162.440001 102.659774) (width 0.5) (layer F.Cu) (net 39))
 (segment (start 192.0725 93.0325) (end 192.29 93.25) (width 0.5) (layer F.Cu) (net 16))
 (segment (start 192.0725 89.875) (end 192.0725 93.0325) (width 0.5) (layer F.Cu) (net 16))
 (segment (start 146.37 112.095) (end 144.305 110.03) (width 0.5) (layer F.Cu) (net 18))
 (segment (start 146.37 116.38) (end 146.37 112.095) (width 0.5) (layer F.Cu) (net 18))
 (segment (start 146.885 112.095) (end 146.37 112.095) (width 0.5) (layer F.Cu) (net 18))
 (segment (start 148.95 110.03) (end 146.885 112.095) (width 0.5) (layer F.Cu) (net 18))
 (segment (start 206.67 83.01) (end 205.07 83.01) (width 0.5) (layer F.Cu) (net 7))
 (segment (start 211.42 87.76) (end 206.67 83.01) (width 0.5) (layer F.Cu) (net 7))
 (segment (start 211.42 90.63) (end 211.42 87.76) (width 0.5) (layer F.Cu) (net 7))
 (segment (start 230.47 105.87) (end 225.39 105.87) (width 0.5) (layer F.Cu) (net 6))
 (segment (start 219.04 98.25) (end 219.04 101.96) (width 0.5) (layer F.Cu) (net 6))
 (segment (start 222.95 105.87) (end 225.39 105.87) (width 0.5) (layer F.Cu) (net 6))
 (segment (start 219.04 101.96) (end 222.95 105.87) (width 0.5) (layer F.Cu) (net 6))
 (segment (start 212.77 115.99) (end 215.78 119) (width 0.5) (layer F.Cu) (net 6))
 (segment (start 212.77 115) (end 212.77 115.99) (width 0.5) (layer F.Cu) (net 6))
 (segment (start 217.550002 119) (end 223 113.550002) (width 0.5) (layer F.Cu) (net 6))
 (segment (start 215.78 119) (end 217.550002 119) (width 0.5) (layer F.Cu) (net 6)))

